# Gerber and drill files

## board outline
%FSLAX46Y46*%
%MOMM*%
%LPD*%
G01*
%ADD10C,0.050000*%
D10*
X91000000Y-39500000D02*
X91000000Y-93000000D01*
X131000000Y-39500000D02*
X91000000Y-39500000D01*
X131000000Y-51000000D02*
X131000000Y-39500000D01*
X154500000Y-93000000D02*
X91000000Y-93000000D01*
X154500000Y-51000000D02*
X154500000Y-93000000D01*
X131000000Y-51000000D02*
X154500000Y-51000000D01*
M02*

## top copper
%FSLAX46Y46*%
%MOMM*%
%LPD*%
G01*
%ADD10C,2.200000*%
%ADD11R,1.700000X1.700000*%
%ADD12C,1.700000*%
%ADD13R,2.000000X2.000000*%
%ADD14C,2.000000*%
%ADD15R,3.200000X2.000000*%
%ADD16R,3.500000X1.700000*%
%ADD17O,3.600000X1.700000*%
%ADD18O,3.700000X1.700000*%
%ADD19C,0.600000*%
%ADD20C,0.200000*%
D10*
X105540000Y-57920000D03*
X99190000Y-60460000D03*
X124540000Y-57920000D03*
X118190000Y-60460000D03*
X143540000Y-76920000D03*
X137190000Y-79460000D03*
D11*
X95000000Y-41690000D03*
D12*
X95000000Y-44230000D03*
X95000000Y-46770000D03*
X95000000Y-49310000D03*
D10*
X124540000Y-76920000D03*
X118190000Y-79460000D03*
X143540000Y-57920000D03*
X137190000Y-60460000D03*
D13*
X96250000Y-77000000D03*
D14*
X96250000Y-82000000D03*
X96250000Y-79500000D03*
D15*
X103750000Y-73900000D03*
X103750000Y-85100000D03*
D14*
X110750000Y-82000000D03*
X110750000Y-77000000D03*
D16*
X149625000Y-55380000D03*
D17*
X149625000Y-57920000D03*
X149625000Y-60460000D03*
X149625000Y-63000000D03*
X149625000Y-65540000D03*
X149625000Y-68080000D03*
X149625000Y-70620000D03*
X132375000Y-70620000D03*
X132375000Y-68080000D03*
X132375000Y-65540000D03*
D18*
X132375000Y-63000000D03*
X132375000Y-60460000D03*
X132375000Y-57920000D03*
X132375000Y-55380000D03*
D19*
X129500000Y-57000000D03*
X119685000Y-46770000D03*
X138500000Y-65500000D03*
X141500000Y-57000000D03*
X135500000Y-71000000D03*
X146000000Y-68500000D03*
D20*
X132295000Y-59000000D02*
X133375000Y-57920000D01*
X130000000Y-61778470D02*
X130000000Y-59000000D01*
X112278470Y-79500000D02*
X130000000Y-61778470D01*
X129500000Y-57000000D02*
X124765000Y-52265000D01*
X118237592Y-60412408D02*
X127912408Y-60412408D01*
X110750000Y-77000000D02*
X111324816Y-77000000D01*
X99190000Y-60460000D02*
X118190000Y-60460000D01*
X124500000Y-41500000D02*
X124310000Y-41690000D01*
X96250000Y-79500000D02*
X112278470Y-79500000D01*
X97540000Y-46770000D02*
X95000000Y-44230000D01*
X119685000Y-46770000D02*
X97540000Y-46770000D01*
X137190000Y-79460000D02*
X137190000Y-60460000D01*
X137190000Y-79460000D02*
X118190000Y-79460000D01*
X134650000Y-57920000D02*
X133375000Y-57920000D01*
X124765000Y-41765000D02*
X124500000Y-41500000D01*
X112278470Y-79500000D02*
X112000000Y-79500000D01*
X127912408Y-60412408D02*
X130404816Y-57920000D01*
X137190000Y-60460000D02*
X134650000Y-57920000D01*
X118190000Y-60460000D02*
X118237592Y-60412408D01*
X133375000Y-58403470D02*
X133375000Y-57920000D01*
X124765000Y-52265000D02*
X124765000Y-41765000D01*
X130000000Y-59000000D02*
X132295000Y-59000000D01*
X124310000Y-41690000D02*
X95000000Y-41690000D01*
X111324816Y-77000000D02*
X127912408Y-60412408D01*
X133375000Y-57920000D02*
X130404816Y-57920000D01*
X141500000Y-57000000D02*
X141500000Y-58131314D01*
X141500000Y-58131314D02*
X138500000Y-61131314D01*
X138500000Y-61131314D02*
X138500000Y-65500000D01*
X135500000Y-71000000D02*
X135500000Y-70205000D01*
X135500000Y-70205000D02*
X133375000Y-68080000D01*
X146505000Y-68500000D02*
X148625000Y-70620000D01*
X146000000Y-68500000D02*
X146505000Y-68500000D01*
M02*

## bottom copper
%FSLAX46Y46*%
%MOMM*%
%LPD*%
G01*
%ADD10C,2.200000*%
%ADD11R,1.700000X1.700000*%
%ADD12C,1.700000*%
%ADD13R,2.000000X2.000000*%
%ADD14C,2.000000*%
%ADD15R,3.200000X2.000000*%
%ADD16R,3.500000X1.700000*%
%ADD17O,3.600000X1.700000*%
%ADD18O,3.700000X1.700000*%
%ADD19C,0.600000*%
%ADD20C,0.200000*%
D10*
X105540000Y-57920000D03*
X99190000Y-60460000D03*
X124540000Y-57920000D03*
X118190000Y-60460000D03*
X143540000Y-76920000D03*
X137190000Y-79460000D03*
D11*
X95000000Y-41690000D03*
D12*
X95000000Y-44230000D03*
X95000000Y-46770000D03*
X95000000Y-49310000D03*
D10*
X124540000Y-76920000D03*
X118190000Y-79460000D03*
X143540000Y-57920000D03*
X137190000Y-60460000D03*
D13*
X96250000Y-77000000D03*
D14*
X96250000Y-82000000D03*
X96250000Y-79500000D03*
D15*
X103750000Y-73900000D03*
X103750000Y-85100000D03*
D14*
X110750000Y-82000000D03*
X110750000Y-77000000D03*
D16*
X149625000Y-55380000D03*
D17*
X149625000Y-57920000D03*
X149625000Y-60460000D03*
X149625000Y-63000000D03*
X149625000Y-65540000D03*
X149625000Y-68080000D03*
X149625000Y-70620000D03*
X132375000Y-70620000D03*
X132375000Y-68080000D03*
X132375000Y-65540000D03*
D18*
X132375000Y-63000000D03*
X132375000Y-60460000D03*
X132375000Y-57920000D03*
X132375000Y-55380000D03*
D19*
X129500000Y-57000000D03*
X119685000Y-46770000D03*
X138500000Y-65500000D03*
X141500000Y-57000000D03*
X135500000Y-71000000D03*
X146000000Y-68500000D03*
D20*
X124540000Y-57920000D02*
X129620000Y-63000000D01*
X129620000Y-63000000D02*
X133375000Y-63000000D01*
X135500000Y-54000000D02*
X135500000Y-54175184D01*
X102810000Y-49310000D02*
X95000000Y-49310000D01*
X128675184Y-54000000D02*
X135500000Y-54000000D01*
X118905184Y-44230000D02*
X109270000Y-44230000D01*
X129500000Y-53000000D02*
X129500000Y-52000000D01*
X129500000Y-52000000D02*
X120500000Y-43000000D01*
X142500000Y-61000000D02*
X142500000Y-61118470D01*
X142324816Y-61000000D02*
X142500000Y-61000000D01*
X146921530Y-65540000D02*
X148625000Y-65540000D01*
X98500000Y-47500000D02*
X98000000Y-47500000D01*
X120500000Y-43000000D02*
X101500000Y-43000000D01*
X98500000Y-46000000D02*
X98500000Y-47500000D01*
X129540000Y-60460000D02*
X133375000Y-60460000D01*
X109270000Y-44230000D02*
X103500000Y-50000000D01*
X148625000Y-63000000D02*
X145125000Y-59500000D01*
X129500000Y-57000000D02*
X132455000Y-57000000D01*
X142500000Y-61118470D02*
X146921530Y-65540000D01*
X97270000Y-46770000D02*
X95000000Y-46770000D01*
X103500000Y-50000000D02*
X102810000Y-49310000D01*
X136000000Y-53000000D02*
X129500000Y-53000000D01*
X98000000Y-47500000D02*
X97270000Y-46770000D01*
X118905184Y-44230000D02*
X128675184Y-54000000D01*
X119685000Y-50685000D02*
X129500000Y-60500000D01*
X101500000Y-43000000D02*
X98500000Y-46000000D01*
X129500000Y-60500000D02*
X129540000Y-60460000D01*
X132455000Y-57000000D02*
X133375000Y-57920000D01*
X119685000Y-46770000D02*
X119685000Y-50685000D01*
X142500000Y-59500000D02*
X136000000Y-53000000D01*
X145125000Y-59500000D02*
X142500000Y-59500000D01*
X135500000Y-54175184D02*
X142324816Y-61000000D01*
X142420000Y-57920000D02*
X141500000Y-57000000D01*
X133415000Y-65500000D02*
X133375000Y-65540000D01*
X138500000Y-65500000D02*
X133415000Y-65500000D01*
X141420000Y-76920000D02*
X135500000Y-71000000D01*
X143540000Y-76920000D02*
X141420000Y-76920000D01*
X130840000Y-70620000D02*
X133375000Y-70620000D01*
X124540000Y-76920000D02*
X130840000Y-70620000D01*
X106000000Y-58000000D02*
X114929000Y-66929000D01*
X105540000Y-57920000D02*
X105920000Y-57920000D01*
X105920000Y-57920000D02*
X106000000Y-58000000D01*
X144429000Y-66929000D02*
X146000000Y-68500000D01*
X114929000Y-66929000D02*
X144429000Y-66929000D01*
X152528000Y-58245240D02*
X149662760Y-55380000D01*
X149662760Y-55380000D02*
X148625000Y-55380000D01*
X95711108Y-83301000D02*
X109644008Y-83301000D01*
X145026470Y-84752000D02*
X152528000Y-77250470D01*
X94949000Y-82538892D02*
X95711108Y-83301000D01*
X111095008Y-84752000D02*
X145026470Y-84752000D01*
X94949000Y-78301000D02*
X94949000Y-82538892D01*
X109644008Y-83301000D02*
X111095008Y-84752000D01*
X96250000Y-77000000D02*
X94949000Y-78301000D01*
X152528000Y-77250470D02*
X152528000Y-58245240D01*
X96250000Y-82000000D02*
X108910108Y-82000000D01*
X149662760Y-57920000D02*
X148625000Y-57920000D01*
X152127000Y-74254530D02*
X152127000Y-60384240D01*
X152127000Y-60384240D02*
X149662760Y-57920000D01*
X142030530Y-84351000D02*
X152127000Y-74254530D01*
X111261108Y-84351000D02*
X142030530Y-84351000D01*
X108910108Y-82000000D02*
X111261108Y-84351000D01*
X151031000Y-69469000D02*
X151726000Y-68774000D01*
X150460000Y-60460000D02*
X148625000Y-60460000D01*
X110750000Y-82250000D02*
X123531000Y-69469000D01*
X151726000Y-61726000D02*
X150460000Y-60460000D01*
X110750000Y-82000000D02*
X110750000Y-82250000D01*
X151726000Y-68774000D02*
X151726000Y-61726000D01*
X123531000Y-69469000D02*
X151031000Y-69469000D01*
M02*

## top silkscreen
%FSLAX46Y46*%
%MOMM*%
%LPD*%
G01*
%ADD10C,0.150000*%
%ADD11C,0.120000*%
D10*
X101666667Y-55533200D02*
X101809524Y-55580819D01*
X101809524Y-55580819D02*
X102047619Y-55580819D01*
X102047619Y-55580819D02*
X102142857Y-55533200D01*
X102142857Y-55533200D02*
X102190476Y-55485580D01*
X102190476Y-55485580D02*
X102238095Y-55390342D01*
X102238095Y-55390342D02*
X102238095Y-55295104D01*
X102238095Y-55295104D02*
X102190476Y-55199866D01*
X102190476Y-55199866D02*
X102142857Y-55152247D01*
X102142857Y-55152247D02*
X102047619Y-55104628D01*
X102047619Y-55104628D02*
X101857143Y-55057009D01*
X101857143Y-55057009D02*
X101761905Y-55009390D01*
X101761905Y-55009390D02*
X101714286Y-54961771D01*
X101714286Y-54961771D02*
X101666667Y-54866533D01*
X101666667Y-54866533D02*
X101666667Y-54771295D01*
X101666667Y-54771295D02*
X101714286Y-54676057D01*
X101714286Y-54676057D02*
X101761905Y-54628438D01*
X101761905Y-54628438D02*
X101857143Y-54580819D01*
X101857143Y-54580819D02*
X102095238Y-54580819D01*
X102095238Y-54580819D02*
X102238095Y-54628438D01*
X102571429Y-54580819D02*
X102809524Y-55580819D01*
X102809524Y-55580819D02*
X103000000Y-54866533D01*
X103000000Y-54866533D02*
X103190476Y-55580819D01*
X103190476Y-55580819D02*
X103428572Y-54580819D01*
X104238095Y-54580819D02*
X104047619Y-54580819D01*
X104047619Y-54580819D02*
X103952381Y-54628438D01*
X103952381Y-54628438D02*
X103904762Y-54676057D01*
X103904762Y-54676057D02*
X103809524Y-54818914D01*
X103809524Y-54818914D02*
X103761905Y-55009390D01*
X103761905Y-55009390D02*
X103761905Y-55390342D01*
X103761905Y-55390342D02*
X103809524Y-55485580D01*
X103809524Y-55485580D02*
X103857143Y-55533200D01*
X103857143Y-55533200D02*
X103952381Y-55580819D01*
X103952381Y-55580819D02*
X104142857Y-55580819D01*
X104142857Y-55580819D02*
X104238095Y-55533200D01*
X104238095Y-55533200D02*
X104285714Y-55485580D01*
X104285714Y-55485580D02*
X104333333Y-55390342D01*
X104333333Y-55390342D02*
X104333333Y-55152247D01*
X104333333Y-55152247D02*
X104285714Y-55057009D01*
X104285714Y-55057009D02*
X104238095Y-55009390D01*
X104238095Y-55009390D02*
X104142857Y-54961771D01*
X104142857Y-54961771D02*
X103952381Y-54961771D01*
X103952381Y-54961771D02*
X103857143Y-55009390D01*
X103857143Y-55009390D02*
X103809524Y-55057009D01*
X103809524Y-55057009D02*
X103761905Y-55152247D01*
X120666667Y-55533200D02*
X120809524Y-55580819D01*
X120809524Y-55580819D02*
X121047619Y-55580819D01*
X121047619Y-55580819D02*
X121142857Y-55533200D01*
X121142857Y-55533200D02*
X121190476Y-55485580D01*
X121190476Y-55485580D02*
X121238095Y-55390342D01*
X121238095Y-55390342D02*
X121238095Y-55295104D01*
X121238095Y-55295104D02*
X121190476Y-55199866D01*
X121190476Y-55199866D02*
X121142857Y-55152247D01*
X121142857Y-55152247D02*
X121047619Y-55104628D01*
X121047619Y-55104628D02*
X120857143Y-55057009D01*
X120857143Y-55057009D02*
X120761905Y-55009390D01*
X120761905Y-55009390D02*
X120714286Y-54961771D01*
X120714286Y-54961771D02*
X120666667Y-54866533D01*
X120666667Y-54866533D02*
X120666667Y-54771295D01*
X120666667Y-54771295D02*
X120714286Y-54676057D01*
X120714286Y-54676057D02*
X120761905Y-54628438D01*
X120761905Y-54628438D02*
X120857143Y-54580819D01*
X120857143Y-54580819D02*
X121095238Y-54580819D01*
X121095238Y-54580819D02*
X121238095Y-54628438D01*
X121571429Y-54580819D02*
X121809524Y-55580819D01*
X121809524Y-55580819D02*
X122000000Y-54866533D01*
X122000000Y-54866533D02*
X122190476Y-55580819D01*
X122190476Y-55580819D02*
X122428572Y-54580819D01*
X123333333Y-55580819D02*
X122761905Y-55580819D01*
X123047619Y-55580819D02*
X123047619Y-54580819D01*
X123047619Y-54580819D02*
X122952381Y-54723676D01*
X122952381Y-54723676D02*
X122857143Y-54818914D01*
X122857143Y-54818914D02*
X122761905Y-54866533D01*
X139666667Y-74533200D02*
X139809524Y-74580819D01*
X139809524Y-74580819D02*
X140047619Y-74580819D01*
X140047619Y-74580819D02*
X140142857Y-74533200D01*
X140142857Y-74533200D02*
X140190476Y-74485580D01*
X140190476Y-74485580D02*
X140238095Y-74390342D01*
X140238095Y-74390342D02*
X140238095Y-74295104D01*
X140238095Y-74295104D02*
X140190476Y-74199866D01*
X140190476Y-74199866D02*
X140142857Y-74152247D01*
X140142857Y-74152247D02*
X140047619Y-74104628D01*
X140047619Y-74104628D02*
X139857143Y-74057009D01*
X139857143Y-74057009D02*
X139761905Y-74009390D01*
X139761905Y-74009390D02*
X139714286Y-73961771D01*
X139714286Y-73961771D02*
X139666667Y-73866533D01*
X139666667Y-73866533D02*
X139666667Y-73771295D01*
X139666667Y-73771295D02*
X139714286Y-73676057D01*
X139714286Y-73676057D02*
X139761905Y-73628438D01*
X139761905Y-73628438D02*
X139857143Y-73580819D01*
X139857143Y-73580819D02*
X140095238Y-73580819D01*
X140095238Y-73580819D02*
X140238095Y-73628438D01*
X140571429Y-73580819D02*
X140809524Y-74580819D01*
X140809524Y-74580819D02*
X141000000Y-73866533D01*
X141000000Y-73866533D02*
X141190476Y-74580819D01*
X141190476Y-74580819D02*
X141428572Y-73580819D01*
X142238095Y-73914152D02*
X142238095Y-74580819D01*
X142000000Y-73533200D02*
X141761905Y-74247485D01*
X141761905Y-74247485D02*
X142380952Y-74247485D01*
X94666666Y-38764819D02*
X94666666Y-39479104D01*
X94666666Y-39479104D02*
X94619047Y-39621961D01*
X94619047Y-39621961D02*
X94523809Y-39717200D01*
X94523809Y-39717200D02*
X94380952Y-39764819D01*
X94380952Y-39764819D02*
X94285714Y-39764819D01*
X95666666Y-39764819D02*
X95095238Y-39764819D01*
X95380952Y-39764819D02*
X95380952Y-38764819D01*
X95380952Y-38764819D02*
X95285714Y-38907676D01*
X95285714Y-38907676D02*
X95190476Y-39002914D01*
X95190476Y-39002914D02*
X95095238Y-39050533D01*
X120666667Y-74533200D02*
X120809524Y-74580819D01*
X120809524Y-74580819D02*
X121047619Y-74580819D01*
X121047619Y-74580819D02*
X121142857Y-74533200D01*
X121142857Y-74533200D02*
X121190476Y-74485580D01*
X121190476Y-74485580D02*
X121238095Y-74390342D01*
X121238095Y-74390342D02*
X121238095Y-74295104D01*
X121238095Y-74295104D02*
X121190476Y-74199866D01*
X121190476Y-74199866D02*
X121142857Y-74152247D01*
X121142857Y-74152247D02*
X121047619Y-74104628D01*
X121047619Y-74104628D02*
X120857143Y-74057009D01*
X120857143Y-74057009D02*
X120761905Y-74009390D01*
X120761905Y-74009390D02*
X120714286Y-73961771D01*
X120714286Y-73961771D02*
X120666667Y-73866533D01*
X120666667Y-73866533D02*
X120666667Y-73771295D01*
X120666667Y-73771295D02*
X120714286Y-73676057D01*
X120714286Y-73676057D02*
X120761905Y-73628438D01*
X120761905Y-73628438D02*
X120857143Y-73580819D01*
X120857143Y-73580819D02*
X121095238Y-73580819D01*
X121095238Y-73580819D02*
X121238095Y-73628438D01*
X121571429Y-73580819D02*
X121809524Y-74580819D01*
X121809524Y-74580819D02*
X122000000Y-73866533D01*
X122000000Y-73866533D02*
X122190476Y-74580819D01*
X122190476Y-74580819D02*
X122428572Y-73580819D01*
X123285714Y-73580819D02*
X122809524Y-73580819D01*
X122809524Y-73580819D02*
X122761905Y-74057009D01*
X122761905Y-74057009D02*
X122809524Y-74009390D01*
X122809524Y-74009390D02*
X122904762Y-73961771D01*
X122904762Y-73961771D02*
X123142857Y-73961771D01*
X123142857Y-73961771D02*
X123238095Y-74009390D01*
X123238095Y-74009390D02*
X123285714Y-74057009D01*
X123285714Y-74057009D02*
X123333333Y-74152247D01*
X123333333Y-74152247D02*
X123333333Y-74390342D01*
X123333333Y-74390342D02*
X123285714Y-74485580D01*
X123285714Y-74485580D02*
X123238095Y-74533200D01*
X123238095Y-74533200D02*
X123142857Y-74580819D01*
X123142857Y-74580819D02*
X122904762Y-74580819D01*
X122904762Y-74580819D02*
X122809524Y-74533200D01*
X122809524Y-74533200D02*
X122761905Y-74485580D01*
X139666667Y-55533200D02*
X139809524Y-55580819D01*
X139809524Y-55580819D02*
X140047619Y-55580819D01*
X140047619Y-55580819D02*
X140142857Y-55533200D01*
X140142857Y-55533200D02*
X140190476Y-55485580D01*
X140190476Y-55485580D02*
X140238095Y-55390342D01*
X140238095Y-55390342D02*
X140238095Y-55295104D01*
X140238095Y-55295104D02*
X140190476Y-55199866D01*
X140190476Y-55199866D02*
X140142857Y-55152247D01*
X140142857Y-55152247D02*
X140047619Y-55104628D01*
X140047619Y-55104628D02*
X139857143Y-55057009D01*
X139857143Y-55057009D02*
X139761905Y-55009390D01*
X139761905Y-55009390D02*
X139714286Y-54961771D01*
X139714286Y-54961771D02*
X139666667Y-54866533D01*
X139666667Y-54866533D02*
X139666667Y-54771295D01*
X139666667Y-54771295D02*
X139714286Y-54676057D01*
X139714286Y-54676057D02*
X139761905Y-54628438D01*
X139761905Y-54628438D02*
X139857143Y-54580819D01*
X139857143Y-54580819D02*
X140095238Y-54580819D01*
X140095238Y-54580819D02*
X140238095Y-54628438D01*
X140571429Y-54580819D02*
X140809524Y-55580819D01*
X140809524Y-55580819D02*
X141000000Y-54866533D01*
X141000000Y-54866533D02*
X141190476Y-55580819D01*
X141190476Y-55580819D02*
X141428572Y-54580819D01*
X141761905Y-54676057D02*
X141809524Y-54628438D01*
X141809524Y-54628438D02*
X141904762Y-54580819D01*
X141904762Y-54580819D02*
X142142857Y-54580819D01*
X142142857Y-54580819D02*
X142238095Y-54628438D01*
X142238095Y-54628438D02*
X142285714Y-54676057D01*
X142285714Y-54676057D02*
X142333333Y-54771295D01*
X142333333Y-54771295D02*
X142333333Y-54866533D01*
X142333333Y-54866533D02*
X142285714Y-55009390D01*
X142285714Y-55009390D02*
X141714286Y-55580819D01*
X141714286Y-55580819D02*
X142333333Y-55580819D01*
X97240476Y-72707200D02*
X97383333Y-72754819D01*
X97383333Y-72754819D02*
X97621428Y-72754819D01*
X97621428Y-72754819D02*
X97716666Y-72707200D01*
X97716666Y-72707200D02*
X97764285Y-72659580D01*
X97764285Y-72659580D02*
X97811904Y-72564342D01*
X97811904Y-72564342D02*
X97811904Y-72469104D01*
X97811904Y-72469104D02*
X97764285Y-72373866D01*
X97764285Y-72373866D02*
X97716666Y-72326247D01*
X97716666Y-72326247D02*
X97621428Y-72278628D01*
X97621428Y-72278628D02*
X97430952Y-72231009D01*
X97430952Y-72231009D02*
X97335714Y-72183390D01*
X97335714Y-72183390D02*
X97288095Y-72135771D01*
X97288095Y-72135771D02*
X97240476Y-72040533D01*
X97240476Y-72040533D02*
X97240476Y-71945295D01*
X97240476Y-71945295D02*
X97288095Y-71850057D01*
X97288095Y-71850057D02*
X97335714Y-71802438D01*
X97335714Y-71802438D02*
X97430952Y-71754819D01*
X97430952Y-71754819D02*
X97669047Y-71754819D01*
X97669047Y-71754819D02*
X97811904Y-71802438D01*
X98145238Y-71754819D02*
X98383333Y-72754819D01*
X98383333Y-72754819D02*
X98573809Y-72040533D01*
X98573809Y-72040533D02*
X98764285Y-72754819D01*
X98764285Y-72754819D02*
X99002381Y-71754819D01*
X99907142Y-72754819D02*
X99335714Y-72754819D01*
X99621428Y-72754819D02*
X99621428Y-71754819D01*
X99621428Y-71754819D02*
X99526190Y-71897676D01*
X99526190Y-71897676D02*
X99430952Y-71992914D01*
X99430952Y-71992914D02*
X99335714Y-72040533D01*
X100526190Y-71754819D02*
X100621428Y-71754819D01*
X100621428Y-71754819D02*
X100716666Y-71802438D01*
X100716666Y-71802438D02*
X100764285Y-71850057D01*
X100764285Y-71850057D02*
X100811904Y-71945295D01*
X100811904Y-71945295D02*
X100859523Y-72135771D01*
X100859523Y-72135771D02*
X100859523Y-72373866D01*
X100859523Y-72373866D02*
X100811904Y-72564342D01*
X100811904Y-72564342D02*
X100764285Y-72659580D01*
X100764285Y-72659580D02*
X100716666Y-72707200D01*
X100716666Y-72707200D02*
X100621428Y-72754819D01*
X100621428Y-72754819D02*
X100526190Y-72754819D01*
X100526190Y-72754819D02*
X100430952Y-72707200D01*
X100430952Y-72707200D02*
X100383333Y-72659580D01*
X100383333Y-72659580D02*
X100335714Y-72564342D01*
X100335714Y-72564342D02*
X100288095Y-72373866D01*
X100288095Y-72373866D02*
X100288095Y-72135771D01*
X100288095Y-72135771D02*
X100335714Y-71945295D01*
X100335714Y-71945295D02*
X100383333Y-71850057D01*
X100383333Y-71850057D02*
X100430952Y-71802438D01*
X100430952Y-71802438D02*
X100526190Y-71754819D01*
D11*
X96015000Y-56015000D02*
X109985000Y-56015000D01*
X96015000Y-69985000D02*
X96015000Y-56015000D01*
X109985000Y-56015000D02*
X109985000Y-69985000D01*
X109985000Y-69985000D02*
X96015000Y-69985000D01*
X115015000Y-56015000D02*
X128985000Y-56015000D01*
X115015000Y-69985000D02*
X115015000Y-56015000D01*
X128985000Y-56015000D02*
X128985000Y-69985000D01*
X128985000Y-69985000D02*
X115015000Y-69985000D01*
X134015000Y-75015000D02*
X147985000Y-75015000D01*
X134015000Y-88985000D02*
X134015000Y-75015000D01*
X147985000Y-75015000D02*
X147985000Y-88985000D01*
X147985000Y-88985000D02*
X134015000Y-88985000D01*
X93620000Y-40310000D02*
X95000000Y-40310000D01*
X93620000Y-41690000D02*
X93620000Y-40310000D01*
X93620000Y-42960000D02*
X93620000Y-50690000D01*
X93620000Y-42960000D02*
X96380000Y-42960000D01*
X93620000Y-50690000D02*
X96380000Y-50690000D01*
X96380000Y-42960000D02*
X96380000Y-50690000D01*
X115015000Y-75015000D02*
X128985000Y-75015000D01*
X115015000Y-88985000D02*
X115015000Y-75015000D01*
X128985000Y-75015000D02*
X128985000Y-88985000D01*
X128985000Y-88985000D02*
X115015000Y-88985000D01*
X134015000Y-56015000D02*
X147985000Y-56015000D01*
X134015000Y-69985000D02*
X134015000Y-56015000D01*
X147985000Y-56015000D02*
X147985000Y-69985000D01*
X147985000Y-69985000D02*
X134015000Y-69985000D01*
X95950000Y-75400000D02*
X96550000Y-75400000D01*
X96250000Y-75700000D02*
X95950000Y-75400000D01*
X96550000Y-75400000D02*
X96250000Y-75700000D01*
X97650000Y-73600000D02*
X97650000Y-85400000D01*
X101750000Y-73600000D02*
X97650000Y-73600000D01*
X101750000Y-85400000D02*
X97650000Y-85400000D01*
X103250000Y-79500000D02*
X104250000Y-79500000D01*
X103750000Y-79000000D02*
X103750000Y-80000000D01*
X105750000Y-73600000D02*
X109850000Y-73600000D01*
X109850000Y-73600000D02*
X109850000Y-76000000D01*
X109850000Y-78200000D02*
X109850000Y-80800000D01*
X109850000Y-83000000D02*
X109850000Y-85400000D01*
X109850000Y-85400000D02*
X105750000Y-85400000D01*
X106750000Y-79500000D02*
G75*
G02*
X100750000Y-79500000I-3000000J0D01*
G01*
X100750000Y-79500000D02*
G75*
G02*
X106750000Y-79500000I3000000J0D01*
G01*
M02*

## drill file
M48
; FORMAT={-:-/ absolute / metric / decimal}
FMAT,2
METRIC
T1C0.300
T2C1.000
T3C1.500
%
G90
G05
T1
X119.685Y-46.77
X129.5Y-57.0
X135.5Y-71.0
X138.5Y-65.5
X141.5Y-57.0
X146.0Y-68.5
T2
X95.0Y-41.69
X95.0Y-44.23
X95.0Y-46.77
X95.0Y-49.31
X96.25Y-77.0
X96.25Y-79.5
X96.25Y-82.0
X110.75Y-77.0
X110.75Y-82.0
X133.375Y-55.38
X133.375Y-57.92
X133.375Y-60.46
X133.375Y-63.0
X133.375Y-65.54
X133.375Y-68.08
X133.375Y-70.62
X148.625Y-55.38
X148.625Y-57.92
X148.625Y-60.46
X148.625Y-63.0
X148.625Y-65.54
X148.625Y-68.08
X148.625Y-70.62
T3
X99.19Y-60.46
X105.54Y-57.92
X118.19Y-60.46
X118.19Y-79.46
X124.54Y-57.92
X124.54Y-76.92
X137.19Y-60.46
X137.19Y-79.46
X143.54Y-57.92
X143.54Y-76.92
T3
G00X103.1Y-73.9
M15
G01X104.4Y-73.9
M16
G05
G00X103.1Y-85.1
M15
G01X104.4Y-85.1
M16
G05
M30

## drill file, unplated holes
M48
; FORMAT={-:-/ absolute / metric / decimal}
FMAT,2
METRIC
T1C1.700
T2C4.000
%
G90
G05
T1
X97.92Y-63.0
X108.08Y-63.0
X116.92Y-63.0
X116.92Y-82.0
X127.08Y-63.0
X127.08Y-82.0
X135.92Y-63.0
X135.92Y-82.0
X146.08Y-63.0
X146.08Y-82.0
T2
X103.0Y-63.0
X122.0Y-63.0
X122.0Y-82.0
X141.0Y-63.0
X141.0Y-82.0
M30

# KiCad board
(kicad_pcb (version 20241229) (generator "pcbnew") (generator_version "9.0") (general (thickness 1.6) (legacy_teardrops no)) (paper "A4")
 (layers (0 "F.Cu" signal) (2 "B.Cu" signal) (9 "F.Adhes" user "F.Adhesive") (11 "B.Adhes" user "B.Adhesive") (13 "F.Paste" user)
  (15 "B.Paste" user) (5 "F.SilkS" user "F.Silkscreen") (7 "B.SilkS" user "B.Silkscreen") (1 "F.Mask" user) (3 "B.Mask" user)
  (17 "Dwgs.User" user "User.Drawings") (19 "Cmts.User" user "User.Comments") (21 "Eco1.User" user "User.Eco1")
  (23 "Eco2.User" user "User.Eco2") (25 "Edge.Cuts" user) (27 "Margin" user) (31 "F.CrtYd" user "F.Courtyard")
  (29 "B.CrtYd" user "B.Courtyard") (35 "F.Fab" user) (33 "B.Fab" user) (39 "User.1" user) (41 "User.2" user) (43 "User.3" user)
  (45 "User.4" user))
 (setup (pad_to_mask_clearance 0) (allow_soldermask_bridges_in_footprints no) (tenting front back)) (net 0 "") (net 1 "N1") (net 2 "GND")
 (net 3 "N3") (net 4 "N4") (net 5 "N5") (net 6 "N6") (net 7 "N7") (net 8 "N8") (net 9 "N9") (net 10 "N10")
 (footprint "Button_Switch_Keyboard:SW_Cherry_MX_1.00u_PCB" (layer "F.Cu") (at 105.54 57.92)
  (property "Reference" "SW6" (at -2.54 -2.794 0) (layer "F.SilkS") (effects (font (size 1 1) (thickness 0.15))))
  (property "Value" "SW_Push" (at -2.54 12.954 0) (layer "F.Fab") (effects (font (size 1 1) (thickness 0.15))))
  (fp_line (start -9.525 -1.905) (end 4.445 -1.905) (stroke (width 0.12) (type solid)) (layer "F.SilkS"))
  (fp_line (start -9.525 12.065) (end -9.525 -1.905) (stroke (width 0.12) (type solid)) (layer "F.SilkS"))
  (fp_line (start 4.445 -1.905) (end 4.445 12.065) (stroke (width 0.12) (type solid)) (layer "F.SilkS"))
  (fp_line (start 4.445 12.065) (end -9.525 12.065) (stroke (width 0.12) (type solid)) (layer "F.SilkS"))
  (pad "" np_thru_hole circle (at -7.62 5.08) (size 1.7 1.7) (drill 1.7) (layers "*.Cu" "*.Mask"))
  (pad "" np_thru_hole circle (at -2.54 5.08) (size 4 4) (drill 4) (layers "*.Cu" "*.Mask"))
  (pad "" np_thru_hole circle (at 2.54 5.08) (size 1.7 1.7) (drill 1.7) (layers "*.Cu" "*.Mask"))
  (pad "1" thru_hole circle (at 0 0) (size 2.2 2.2) (drill 1.5) (layers "*.Cu" "*.Mask") (remove_unused_layers no) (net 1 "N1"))
  (pad "2" thru_hole circle (at -6.35 2.54) (size 2.2 2.2) (drill 1.5) (layers "*.Cu" "*.Mask") (remove_unused_layers no) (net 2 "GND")))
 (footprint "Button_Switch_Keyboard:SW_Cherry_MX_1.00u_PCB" (layer "F.Cu") (at 124.54 57.92)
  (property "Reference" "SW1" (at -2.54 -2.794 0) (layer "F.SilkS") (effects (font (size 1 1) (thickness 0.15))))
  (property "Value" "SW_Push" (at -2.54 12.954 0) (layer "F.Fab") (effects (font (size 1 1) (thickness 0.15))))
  (fp_line (start -9.525 -1.905) (end 4.445 -1.905) (stroke (width 0.12) (type solid)) (layer "F.SilkS"))
  (fp_line (start -9.525 12.065) (end -9.525 -1.905) (stroke (width 0.12) (type solid)) (layer "F.SilkS"))
  (fp_line (start 4.445 -1.905) (end 4.445 12.065) (stroke (width 0.12) (type solid)) (layer "F.SilkS"))
  (fp_line (start 4.445 12.065) (end -9.525 12.065) (stroke (width 0.12) (type solid)) (layer "F.SilkS"))
  (pad "" np_thru_hole circle (at -7.62 5.08) (size 1.7 1.7) (drill 1.7) (layers "*.Cu" "*.Mask"))
  (pad "" np_thru_hole circle (at -2.54 5.08) (size 4 4) (drill 4) (layers "*.Cu" "*.Mask"))
  (pad "" np_thru_hole circle (at 2.54 5.08) (size 1.7 1.7) (drill 1.7) (layers "*.Cu" "*.Mask"))
  (pad "1" thru_hole circle (at 0 0) (size 2.2 2.2) (drill 1.5) (layers "*.Cu" "*.Mask") (remove_unused_layers no) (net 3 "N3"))
  (pad "2" thru_hole circle (at -6.35 2.54) (size 2.2 2.2) (drill 1.5) (layers "*.Cu" "*.Mask") (remove_unused_layers no) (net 2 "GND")))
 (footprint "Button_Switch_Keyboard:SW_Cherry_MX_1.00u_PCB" (layer "F.Cu") (at 143.54 76.92)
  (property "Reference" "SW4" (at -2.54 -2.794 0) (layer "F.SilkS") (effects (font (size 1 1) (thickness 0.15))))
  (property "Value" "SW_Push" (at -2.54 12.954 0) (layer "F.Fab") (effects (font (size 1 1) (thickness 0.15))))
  (fp_line (start -9.525 -1.905) (end 4.445 -1.905) (stroke (width 0.12) (type solid)) (layer "F.SilkS"))
  (fp_line (start -9.525 12.065) (end -9.525 -1.905) (stroke (width 0.12) (type solid)) (layer "F.SilkS"))
  (fp_line (start 4.445 -1.905) (end 4.445 12.065) (stroke (width 0.12) (type solid)) (layer "F.SilkS"))
  (fp_line (start 4.445 12.065) (end -9.525 12.065) (stroke (width 0.12) (type solid)) (layer "F.SilkS"))
  (pad "" np_thru_hole circle (at -7.62 5.08) (size 1.7 1.7) (drill 1.7) (layers "*.Cu" "*.Mask"))
  (pad "" np_thru_hole circle (at -2.54 5.08) (size 4 4) (drill 4) (layers "*.Cu" "*.Mask"))
  (pad "" np_thru_hole circle (at 2.54 5.08) (size 1.7 1.7) (drill 1.7) (layers "*.Cu" "*.Mask"))
  (pad "1" thru_hole circle (at 0 0) (size 2.2 2.2) (drill 1.5) (layers "*.Cu" "*.Mask") (remove_unused_layers no) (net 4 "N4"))
  (pad "2" thru_hole circle (at -6.35 2.54) (size 2.2 2.2) (drill 1.5) (layers "*.Cu" "*.Mask") (remove_unused_layers no) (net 2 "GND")))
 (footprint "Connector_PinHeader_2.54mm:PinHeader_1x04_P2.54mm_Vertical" (layer "F.Cu") (at 95 41.69)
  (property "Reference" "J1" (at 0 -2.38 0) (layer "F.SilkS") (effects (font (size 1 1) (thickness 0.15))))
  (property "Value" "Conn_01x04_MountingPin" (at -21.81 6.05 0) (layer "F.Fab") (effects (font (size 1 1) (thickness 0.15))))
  (fp_line (start -1.38 -1.38) (end 0 -1.38) (stroke (width 0.12) (type solid)) (layer "F.SilkS"))
  (fp_line (start -1.38 0) (end -1.38 -1.38) (stroke (width 0.12) (type solid)) (layer "F.SilkS"))
  (fp_line (start -1.38 1.27) (end -1.38 9) (stroke (width 0.12) (type solid)) (layer "F.SilkS"))
  (fp_line (start -1.38 1.27) (end 1.38 1.27) (stroke (width 0.12) (type solid)) (layer "F.SilkS"))
  (fp_line (start -1.38 9) (end 1.38 9) (stroke (width 0.12) (type solid)) (layer "F.SilkS"))
  (fp_line (start 1.38 1.27) (end 1.38 9) (stroke (width 0.12) (type solid)) (layer "F.SilkS"))
  (pad "1" thru_hole rect (at 0 0) (size 1.7 1.7) (drill 1) (layers "*.Cu" "*.Mask") (remove_unused_layers no) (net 2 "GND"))
  (pad "2" thru_hole circle (at 0 2.54) (size 1.7 1.7) (drill 1) (layers "*.Cu" "*.Mask") (remove_unused_layers no) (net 2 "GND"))
  (pad "3" thru_hole circle (at 0 5.08) (size 1.7 1.7) (drill 1) (layers "*.Cu" "*.Mask") (remove_unused_layers no) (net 2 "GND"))
  (pad "4" thru_hole circle (at 0 7.62) (size 1.7 1.7) (drill 1) (layers "*.Cu" "*.Mask") (remove_unused_layers no) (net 2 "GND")))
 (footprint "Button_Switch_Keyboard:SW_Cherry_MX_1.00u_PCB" (layer "F.Cu") (at 124.54 76.92)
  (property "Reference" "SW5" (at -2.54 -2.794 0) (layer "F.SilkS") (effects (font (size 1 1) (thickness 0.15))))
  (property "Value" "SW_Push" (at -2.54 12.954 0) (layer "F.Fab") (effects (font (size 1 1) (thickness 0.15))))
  (fp_line (start -9.525 -1.905) (end 4.445 -1.905) (stroke (width 0.12) (type solid)) (layer "F.SilkS"))
  (fp_line (start -9.525 12.065) (end -9.525 -1.905) (stroke (width 0.12) (type solid)) (layer "F.SilkS"))
  (fp_line (start 4.445 -1.905) (end 4.445 12.065) (stroke (width 0.12) (type solid)) (layer "F.SilkS"))
  (fp_line (start 4.445 12.065) (end -9.525 12.065) (stroke (width 0.12) (type solid)) (layer "F.SilkS"))
  (pad "" np_thru_hole circle (at -7.62 5.08) (size 1.7 1.7) (drill 1.7) (layers "*.Cu" "*.Mask"))
  (pad "" np_thru_hole circle (at -2.54 5.08) (size 4 4) (drill 4) (layers "*.Cu" "*.Mask"))
  (pad "" np_thru_hole circle (at 2.54 5.08) (size 1.7 1.7) (drill 1.7) (layers "*.Cu" "*.Mask"))
  (pad "1" thru_hole circle (at 0 0) (size 2.2 2.2) (drill 1.5) (layers "*.Cu" "*.Mask") (remove_unused_layers no) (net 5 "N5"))
  (pad "2" thru_hole circle (at -6.35 2.54) (size 2.2 2.2) (drill 1.5) (layers "*.Cu" "*.Mask") (remove_unused_layers no) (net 2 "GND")))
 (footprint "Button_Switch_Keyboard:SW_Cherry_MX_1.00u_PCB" (layer "F.Cu") (at 143.54 57.92)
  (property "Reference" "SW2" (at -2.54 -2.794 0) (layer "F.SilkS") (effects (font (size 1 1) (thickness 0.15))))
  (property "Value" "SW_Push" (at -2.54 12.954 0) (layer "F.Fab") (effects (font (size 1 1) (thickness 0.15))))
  (fp_line (start -9.525 -1.905) (end 4.445 -1.905) (stroke (width 0.12) (type solid)) (layer "F.SilkS"))
  (fp_line (start -9.525 12.065) (end -9.525 -1.905) (stroke (width 0.12) (type solid)) (layer "F.SilkS"))
  (fp_line (start 4.445 -1.905) (end 4.445 12.065) (stroke (width 0.12) (type solid)) (layer "F.SilkS"))
  (fp_line (start 4.445 12.065) (end -9.525 12.065) (stroke (width 0.12) (type solid)) (layer "F.SilkS"))
  (pad "" np_thru_hole circle (at -7.62 5.08) (size 1.7 1.7) (drill 1.7) (layers "*.Cu" "*.Mask"))
  (pad "" np_thru_hole circle (at -2.54 5.08) (size 4 4) (drill 4) (layers "*.Cu" "*.Mask"))
  (pad "" np_thru_hole circle (at 2.54 5.08) (size 1.7 1.7) (drill 1.7) (layers "*.Cu" "*.Mask"))
  (pad "1" thru_hole circle (at 0 0) (size 2.2 2.2) (drill 1.5) (layers "*.Cu" "*.Mask") (remove_unused_layers no) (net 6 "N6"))
  (pad "2" thru_hole circle (at -6.35 2.54) (size 2.2 2.2) (drill 1.5) (layers "*.Cu" "*.Mask") (remove_unused_layers no) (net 2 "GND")))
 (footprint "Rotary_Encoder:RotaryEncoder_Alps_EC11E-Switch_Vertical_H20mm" (layer "F.Cu") (at 96.25 77)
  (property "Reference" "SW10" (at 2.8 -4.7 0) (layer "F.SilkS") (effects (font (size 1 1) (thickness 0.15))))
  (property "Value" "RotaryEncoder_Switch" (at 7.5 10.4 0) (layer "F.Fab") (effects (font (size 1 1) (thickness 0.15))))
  (fp_line (start -0.3 -1.6) (end 0.3 -1.6) (stroke (width 0.12) (type solid)) (layer "F.SilkS"))
  (fp_line (start 0 -1.3) (end -0.3 -1.6) (stroke (width 0.12) (type solid)) (layer "F.SilkS"))
  (fp_line (start 0.3 -1.6) (end 0 -1.3) (stroke (width 0.12) (type solid)) (layer "F.SilkS"))
  (fp_line (start 1.4 -3.4) (end 1.4 8.4) (stroke (width 0.12) (type solid)) (layer "F.SilkS"))
  (fp_line (start 5.5 -3.4) (end 1.4 -3.4) (stroke (width 0.12) (type solid)) (layer "F.SilkS"))
  (fp_line (start 5.5 8.4) (end 1.4 8.4) (stroke (width 0.12) (type solid)) (layer "F.SilkS"))
  (fp_line (start 7 2.5) (end 8 2.5) (stroke (width 0.12) (type solid)) (layer "F.SilkS"))
  (fp_line (start 7.5 2) (end 7.5 3) (stroke (width 0.12) (type solid)) (layer "F.SilkS"))
  (fp_line (start 9.5 -3.4) (end 13.6 -3.4) (stroke (width 0.12) (type solid)) (layer "F.SilkS"))
  (fp_line (start 13.6 -3.4) (end 13.6 -1) (stroke (width 0.12) (type solid)) (layer "F.SilkS"))
  (fp_line (start 13.6 1.2) (end 13.6 3.8) (stroke (width 0.12) (type solid)) (layer "F.SilkS"))
  (fp_line (start 13.6 6) (end 13.6 8.4) (stroke (width 0.12) (type solid)) (layer "F.SilkS"))
  (fp_line (start 13.6 8.4) (end 9.5 8.4) (stroke (width 0.12) (type solid)) (layer "F.SilkS"))
  (fp_circle (center 7.5 2.5) (end 10.5 2.5) (stroke (width 0.12) (type solid)) (fill no) (layer "F.SilkS"))
  (pad "A" thru_hole rect (at 0 0) (size 2 2) (drill 1) (layers "*.Cu" "*.Mask") (remove_unused_layers no) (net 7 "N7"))
  (pad "B" thru_hole circle (at 0 5) (size 2 2) (drill 1) (layers "*.Cu" "*.Mask") (remove_unused_layers no) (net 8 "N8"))
  (pad "C" thru_hole circle (at 0 2.5) (size 2 2) (drill 1) (layers "*.Cu" "*.Mask") (remove_unused_layers no) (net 2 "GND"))
  (pad "MP" thru_hole rect (at 7.5 -3.1) (size 3.2 2) (drill oval 2.8 1.5) (layers "*.Cu" "*.Mask") (remove_unused_layers no))
  (pad "MP" thru_hole rect (at 7.5 8.1) (size 3.2 2) (drill oval 2.8 1.5) (layers "*.Cu" "*.Mask") (remove_unused_layers no))
  (pad "S1" thru_hole circle (at 14.5 5) (size 2 2) (drill 1) (layers "*.Cu" "*.Mask") (remove_unused_layers no) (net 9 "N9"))
  (pad "S2" thru_hole circle (at 14.5 0) (size 2 2) (drill 1) (layers "*.Cu" "*.Mask") (remove_unused_layers no) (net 2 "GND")))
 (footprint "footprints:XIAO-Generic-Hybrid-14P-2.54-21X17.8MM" (layer "B.Cu") (at 141 63 180)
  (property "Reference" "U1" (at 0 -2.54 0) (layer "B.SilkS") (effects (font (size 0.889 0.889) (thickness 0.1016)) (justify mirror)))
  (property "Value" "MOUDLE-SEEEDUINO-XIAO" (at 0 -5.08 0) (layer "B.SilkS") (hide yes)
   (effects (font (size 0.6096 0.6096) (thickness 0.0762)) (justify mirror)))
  (pad "1" thru_hole rect (at -7.625 7.62 180) (size 3.5 1.7) (drill 1 (offset -1 0)) (layers "*.Cu" "*.Mask") (remove_unused_layers no)
   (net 7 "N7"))
  (pad "2" thru_hole oval (at -7.625 5.08 180) (size 3.6 1.7) (drill 1 (offset -1 0)) (layers "*.Cu" "*.Mask") (remove_unused_layers no)
   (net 8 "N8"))
  (pad "3" thru_hole oval (at -7.625 2.54 180) (size 3.6 1.7) (drill 1 (offset -1 0)) (layers "*.Cu" "*.Mask") (remove_unused_layers no)
   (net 9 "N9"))
  (pad "4" thru_hole oval (at -7.625 0 180) (size 3.6 1.7) (drill 1 (offset -1 0)) (layers "*.Cu" "*.Mask") (remove_unused_layers no)
   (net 2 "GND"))
  (pad "5" thru_hole oval (at -7.625 -2.54 180) (size 3.6 1.7) (drill 1 (offset -1 0)) (layers "*.Cu" "*.Mask") (remove_unused_layers no)
   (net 2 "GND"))
  (pad "6" thru_hole oval (at -7.625 -5.08) (size 3.6 1.7) (drill 1 (offset 1 0)) (layers "*.Cu" "*.Mask") (remove_unused_layers no)
   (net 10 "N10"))
  (pad "7" thru_hole oval (at -7.625 -7.62 180) (size 3.6 1.7) (drill 1 (offset -1 0)) (layers "*.Cu" "*.Mask") (remove_unused_layers no)
   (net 1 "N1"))
  (pad "8" thru_hole oval (at 7.625 -7.62 180) (size 3.6 1.7) (drill 1 (offset 1 0)) (layers "*.Cu" "*.Mask") (remove_unused_layers no)
   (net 5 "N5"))
  (pad "9" thru_hole oval (at 7.625 -5.08 180) (size 3.6 1.7) (drill 1 (offset 1 0)) (layers "*.Cu" "*.Mask") (remove_unused_layers no)
   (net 4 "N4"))
  (pad "10" thru_hole oval (at 7.625 -2.54 180) (size 3.6 1.7) (drill 1 (offset 1 0)) (layers "*.Cu" "*.Mask") (remove_unused_layers no)
   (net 6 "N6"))
  (pad "11" thru_hole oval (at 7.625 0 180) (size 3.7 1.7) (drill 1 (offset 1 0)) (layers "*.Cu" "*.Mask") (remove_unused_layers no)
   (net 3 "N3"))
  (pad "12" thru_hole oval (at 7.625 2.54 180) (size 3.7 1.7) (drill 1 (offset 1 0)) (layers "*.Cu" "*.Mask") (remove_unused_layers no)
   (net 2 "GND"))
  (pad "13" thru_hole oval (at 7.625 5.08 180) (size 3.7 1.7) (drill 1 (offset 1 0)) (layers "*.Cu" "*.Mask") (remove_unused_layers no)
   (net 2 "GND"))
  (pad "14" thru_hole oval (at 7.625 7.62 180) (size 3.7 1.7) (drill 1 (offset 1 0)) (layers "*.Cu" "*.Mask") (remove_unused_layers no)
   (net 2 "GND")))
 (gr_line (start 154.5 93) (end 91 93) (stroke (width 0.05) (type default)) (layer "Edge.Cuts"))
 (gr_line (start 154.5 51) (end 154.5 93) (stroke (width 0.05) (type default)) (layer "Edge.Cuts"))
 (gr_line (start 91 39.5) (end 91 93) (stroke (width 0.05) (type default)) (layer "Edge.Cuts"))
 (gr_line (start 131 51) (end 131 39.5) (stroke (width 0.05) (type default)) (layer "Edge.Cuts"))
 (gr_line (start 131 51) (end 154.5 51) (stroke (width 0.05) (type default)) (layer "Edge.Cuts"))
 (gr_line (start 131 39.5) (end 91 39.5) (stroke (width 0.05) (type default)) (layer "Edge.Cuts"))
 (segment (start 124.54 57.92) (end 129.62 63) (width 0.2) (layer "B.Cu") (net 3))
 (segment (start 129.62 63) (end 133.375 63) (width 0.2) (layer "B.Cu") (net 3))
 (segment (start 132.295 59) (end 133.375 57.92) (width 0.2) (layer "F.Cu") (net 2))
 (segment (start 130 61.77847) (end 130 59) (width 0.2) (layer "F.Cu") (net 2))
 (segment (start 112.27847 79.5) (end 130 61.77847) (width 0.2) (layer "F.Cu") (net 2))
 (segment (start 129.5 57) (end 124.765 52.265) (width 0.2) (layer "F.Cu") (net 2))
 (segment (start 118.237592 60.412408) (end 127.912408 60.412408) (width 0.2) (layer "F.Cu") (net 2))
 (segment (start 110.75 77) (end 111.324816 77) (width 0.2) (layer "F.Cu") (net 2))
 (segment (start 99.19 60.46) (end 118.19 60.46) (width 0.2) (layer "F.Cu") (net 2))
 (segment (start 124.5 41.5) (end 124.31 41.69) (width 0.2) (layer "F.Cu") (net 2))
 (segment (start 96.25 79.5) (end 112.27847 79.5) (width 0.2) (layer "F.Cu") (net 2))
 (segment (start 97.54 46.77) (end 95 44.23) (width 0.2) (layer "F.Cu") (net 2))
 (segment (start 119.685 46.77) (end 97.54 46.77) (width 0.2) (layer "F.Cu") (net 2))
 (segment (start 137.19 79.46) (end 137.19 60.46) (width 0.2) (layer "F.Cu") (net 2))
 (segment (start 137.19 79.46) (end 118.19 79.46) (width 0.2) (layer "F.Cu") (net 2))
 (segment (start 134.65 57.92) (end 133.375 57.92) (width 0.2) (layer "F.Cu") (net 2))
 (segment (start 124.765 41.765) (end 124.5 41.5) (width 0.2) (layer "F.Cu") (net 2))
 (segment (start 112.27847 79.5) (end 112 79.5) (width 0.2) (layer "F.Cu") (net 2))
 (segment (start 127.912408 60.412408) (end 130.404816 57.92) (width 0.2) (layer "F.Cu") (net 2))
 (segment (start 137.19 60.46) (end 134.65 57.92) (width 0.2) (layer "F.Cu") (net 2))
 (segment (start 118.19 60.46) (end 118.237592 60.412408) (width 0.2) (layer "F.Cu") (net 2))
 (segment (start 133.375 58.40347) (end 133.375 57.92) (width 0.2) (layer "F.Cu") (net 2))
 (segment (start 124.765 52.265) (end 124.765 41.765) (width 0.2) (layer "F.Cu") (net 2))
 (segment (start 130 59) (end 132.295 59) (width 0.2) (layer "F.Cu") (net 2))
 (segment (start 124.31 41.69) (end 95 41.69) (width 0.2) (layer "F.Cu") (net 2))
 (segment (start 111.324816 77) (end 127.912408 60.412408) (width 0.2) (layer "F.Cu") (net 2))
 (segment (start 133.375 57.92) (end 130.404816 57.92) (width 0.2) (layer "F.Cu") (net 2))
 (via (at 129.5 57) (size 0.6) (drill 0.3) (layers "F.Cu" "B.Cu") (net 2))
 (via (at 119.685 46.77) (size 0.6) (drill 0.3) (layers "F.Cu" "B.Cu") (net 2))
 (segment (start 135.5 54) (end 135.5 54.175184) (width 0.2) (layer "B.Cu") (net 2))
 (segment (start 102.81 49.31) (end 95 49.31) (width 0.2) (layer "B.Cu") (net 2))
 (segment (start 128.675184 54) (end 135.5 54) (width 0.2) (layer "B.Cu") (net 2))
 (segment (start 118.905184 44.23) (end 109.27 44.23) (width 0.2) (layer "B.Cu") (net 2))
 (segment (start 129.5 53) (end 129.5 52) (width 0.2) (layer "B.Cu") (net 2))
 (segment (start 129.5 52) (end 120.5 43) (width 0.2) (layer "B.Cu") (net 2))
 (segment (start 142.5 61) (end 142.5 61.11847) (width 0.2) (layer "B.Cu") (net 2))
 (segment (start 142.324816 61) (end 142.5 61) (width 0.2) (layer "B.Cu") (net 2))
 (segment (start 146.92153 65.54) (end 148.625 65.54) (width 0.2) (layer "B.Cu") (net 2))
 (segment (start 98.5 47.5) (end 98 47.5) (width 0.2) (layer "B.Cu") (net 2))
 (segment (start 120.5 43) (end 101.5 43) (width 0.2) (layer "B.Cu") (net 2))
 (segment (start 98.5 46) (end 98.5 47.5) (width 0.2) (layer "B.Cu") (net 2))
 (segment (start 129.54 60.46) (end 133.375 60.46) (width 0.2) (layer "B.Cu") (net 2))
 (segment (start 109.27 44.23) (end 103.5 50) (width 0.2) (layer "B.Cu") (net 2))
 (segment (start 148.625 63) (end 145.125 59.5) (width 0.2) (layer "B.Cu") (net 2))
 (segment (start 129.5 57) (end 132.455 57) (width 0.2) (layer "B.Cu") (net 2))
 (segment (start 142.5 61.11847) (end 146.92153 65.54) (width 0.2) (layer "B.Cu") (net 2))
 (segment (start 97.27 46.77) (end 95 46.77) (width 0.2) (layer "B.Cu") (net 2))
 (segment (start 103.5 50) (end 102.81 49.31) (width 0.2) (layer "B.Cu") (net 2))
 (segment (start 136 53) (end 129.5 53) (width 0.2) (layer "B.Cu") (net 2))
 (segment (start 98 47.5) (end 97.27 46.77) (width 0.2) (layer "B.Cu") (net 2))
 (segment (start 118.905184 44.23) (end 128.675184 54) (width 0.2) (layer "B.Cu") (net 2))
 (segment (start 119.685 50.685) (end 129.5 60.5) (width 0.2) (layer "B.Cu") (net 2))
 (segment (start 101.5 43) (end 98.5 46) (width 0.2) (layer "B.Cu") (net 2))
 (segment (start 129.5 60.5) (end 129.54 60.46) (width 0.2) (layer "B.Cu") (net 2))
 (segment (start 132.455 57) (end 133.375 57.92) (width 0.2) (layer "B.Cu") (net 2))
 (segment (start 119.685 46.77) (end 119.685 50.685) (width 0.2) (layer "B.Cu") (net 2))
 (segment (start 142.5 59.5) (end 136 53) (width 0.2) (layer "B.Cu") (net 2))
 (segment (start 145.125 59.5) (end 142.5 59.5) (width 0.2) (layer "B.Cu") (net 2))
 (segment (start 135.5 54.175184) (end 142.324816 61) (width 0.2) (layer "B.Cu") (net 2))
 (segment (start 141.5 57) (end 141.5 58.131314) (width 0.2) (layer "F.Cu") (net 6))
 (segment (start 141.5 58.131314) (end 138.5 61.131314) (width 0.2) (layer "F.Cu") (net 6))
 (segment (start 138.5 61.131314) (end 138.5 65.5) (width 0.2) (layer "F.Cu") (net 6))
 (via (at 138.5 65.5) (size 0.6) (drill 0.3) (layers "F.Cu" "B.Cu") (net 6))
 (via (at 141.5 57) (size 0.6) (drill 0.3) (layers "F.Cu" "B.Cu") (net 6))
 (segment (start 142.42 57.92) (end 141.5 57) (width 0.2) (layer "B.Cu") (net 6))
 (segment (start 133.415 65.5) (end 133.375 65.54) (width 0.2) (layer "B.Cu") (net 6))
 (segment (start 138.5 65.5) (end 133.415 65.5) (width 0.2) (layer "B.Cu") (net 6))
 (segment (start 135.5 71) (end 135.5 70.205) (width 0.2) (layer "F.Cu") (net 4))
 (segment (start 135.5 70.205) (end 133.375 68.08) (width 0.2) (layer "F.Cu") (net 4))
 (via (at 135.5 71) (size 0.6) (drill 0.3) (layers "F.Cu" "B.Cu") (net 4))
 (segment (start 141.42 76.92) (end 135.5 71) (width 0.2) (layer "B.Cu") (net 4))
 (segment (start 143.54 76.92) (end 141.42 76.92) (width 0.2) (layer "B.Cu") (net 4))
 (segment (start 130.84 70.62) (end 133.375 70.62) (width 0.2) (layer "B.Cu") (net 5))
 (segment (start 124.54 76.92) (end 130.84 70.62) (width 0.2) (layer "B.Cu") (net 5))
 (segment (start 146.505 68.5) (end 148.625 70.62) (width 0.2) (layer "F.Cu") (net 1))
 (segment (start 146 68.5) (end 146.505 68.5) (width 0.2) (layer "F.Cu") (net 1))
 (via (at 146 68.5) (size 0.6) (drill 0.3) (layers "F.Cu" "B.Cu") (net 1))
 (segment (start 106 58) (end 114.929 66.929) (width 0.2) (layer "B.Cu") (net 1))
 (segment (start 105.54 57.92) (end 105.92 57.92) (width 0.2) (layer "B.Cu") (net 1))
 (segment (start 105.92 57.92) (end 106 58) (width 0.2) (layer "B.Cu") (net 1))
 (segment (start 144.429 66.929) (end 146 68.5) (width 0.2) (layer "B.Cu") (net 1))
 (segment (start 114.929 66.929) (end 144.429 66.929) (width 0.2) (layer "B.Cu") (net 1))
 (segment (start 152.528 58.24524) (end 149.66276 55.38) (width 0.2) (layer "B.Cu") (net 7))
 (segment (start 149.66276 55.38) (end 148.625 55.38) (width 0.2) (layer "B.Cu") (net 7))
 (segment (start 95.711108 83.301) (end 109.644008 83.301) (width 0.2) (layer "B.Cu") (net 7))
 (segment (start 145.02647 84.752) (end 152.528 77.25047) (width 0.2) (layer "B.Cu") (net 7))
 (segment (start 94.949 82.538892) (end 95.711108 83.301) (width 0.2) (layer "B.Cu") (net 7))
 (segment (start 111.095008 84.752) (end 145.02647 84.752) (width 0.2) (layer "B.Cu") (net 7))
 (segment (start 94.949 78.301) (end 94.949 82.538892) (width 0.2) (layer "B.Cu") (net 7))
 (segment (start 109.644008 83.301) (end 111.095008 84.752) (width 0.2) (layer "B.Cu") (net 7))
 (segment (start 96.25 77) (end 94.949 78.301) (width 0.2) (layer "B.Cu") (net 7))
 (segment (start 152.528 77.25047) (end 152.528 58.24524) (width 0.2) (layer "B.Cu") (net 7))
 (segment (start 96.25 82) (end 108.910108 82) (width 0.2) (layer "B.Cu") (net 8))
 (segment (start 149.66276 57.92) (end 148.625 57.92) (width 0.2) (layer "B.Cu") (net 8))
 (segment (start 152.127 74.25453) (end 152.127 60.38424) (width 0.2) (layer "B.Cu") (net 8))
 (segment (start 152.127 60.38424) (end 149.66276 57.92) (width 0.2) (layer "B.Cu") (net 8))
 (segment (start 142.03053 84.351) (end 152.127 74.25453) (width 0.2) (layer "B.Cu") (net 8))
 (segment (start 111.261108 84.351) (end 142.03053 84.351) (width 0.2) (layer "B.Cu") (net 8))
 (segment (start 108.910108 82) (end 111.261108 84.351) (width 0.2) (layer "B.Cu") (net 8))
 (segment (start 151.031 69.469) (end 151.726 68.774) (width 0.2) (layer "B.Cu") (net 9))
 (segment (start 150.46 60.46) (end 148.625 60.46) (width 0.2) (layer "B.Cu") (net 9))
 (segment (start 110.75 82.25) (end 123.531 69.469) (width 0.2) (layer "B.Cu") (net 9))
 (segment (start 151.726 61.726) (end 150.46 60.46) (width 0.2) (layer "B.Cu") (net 9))
 (segment (start 110.75 82) (end 110.75 82.25) (width 0.2) (layer "B.Cu") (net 9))
 (segment (start 151.726 68.774) (end 151.726 61.726) (width 0.2) (layer "B.Cu") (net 9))
 (segment (start 123.531 69.469) (end 151.031 69.469) (width 0.2) (layer "B.Cu") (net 9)))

